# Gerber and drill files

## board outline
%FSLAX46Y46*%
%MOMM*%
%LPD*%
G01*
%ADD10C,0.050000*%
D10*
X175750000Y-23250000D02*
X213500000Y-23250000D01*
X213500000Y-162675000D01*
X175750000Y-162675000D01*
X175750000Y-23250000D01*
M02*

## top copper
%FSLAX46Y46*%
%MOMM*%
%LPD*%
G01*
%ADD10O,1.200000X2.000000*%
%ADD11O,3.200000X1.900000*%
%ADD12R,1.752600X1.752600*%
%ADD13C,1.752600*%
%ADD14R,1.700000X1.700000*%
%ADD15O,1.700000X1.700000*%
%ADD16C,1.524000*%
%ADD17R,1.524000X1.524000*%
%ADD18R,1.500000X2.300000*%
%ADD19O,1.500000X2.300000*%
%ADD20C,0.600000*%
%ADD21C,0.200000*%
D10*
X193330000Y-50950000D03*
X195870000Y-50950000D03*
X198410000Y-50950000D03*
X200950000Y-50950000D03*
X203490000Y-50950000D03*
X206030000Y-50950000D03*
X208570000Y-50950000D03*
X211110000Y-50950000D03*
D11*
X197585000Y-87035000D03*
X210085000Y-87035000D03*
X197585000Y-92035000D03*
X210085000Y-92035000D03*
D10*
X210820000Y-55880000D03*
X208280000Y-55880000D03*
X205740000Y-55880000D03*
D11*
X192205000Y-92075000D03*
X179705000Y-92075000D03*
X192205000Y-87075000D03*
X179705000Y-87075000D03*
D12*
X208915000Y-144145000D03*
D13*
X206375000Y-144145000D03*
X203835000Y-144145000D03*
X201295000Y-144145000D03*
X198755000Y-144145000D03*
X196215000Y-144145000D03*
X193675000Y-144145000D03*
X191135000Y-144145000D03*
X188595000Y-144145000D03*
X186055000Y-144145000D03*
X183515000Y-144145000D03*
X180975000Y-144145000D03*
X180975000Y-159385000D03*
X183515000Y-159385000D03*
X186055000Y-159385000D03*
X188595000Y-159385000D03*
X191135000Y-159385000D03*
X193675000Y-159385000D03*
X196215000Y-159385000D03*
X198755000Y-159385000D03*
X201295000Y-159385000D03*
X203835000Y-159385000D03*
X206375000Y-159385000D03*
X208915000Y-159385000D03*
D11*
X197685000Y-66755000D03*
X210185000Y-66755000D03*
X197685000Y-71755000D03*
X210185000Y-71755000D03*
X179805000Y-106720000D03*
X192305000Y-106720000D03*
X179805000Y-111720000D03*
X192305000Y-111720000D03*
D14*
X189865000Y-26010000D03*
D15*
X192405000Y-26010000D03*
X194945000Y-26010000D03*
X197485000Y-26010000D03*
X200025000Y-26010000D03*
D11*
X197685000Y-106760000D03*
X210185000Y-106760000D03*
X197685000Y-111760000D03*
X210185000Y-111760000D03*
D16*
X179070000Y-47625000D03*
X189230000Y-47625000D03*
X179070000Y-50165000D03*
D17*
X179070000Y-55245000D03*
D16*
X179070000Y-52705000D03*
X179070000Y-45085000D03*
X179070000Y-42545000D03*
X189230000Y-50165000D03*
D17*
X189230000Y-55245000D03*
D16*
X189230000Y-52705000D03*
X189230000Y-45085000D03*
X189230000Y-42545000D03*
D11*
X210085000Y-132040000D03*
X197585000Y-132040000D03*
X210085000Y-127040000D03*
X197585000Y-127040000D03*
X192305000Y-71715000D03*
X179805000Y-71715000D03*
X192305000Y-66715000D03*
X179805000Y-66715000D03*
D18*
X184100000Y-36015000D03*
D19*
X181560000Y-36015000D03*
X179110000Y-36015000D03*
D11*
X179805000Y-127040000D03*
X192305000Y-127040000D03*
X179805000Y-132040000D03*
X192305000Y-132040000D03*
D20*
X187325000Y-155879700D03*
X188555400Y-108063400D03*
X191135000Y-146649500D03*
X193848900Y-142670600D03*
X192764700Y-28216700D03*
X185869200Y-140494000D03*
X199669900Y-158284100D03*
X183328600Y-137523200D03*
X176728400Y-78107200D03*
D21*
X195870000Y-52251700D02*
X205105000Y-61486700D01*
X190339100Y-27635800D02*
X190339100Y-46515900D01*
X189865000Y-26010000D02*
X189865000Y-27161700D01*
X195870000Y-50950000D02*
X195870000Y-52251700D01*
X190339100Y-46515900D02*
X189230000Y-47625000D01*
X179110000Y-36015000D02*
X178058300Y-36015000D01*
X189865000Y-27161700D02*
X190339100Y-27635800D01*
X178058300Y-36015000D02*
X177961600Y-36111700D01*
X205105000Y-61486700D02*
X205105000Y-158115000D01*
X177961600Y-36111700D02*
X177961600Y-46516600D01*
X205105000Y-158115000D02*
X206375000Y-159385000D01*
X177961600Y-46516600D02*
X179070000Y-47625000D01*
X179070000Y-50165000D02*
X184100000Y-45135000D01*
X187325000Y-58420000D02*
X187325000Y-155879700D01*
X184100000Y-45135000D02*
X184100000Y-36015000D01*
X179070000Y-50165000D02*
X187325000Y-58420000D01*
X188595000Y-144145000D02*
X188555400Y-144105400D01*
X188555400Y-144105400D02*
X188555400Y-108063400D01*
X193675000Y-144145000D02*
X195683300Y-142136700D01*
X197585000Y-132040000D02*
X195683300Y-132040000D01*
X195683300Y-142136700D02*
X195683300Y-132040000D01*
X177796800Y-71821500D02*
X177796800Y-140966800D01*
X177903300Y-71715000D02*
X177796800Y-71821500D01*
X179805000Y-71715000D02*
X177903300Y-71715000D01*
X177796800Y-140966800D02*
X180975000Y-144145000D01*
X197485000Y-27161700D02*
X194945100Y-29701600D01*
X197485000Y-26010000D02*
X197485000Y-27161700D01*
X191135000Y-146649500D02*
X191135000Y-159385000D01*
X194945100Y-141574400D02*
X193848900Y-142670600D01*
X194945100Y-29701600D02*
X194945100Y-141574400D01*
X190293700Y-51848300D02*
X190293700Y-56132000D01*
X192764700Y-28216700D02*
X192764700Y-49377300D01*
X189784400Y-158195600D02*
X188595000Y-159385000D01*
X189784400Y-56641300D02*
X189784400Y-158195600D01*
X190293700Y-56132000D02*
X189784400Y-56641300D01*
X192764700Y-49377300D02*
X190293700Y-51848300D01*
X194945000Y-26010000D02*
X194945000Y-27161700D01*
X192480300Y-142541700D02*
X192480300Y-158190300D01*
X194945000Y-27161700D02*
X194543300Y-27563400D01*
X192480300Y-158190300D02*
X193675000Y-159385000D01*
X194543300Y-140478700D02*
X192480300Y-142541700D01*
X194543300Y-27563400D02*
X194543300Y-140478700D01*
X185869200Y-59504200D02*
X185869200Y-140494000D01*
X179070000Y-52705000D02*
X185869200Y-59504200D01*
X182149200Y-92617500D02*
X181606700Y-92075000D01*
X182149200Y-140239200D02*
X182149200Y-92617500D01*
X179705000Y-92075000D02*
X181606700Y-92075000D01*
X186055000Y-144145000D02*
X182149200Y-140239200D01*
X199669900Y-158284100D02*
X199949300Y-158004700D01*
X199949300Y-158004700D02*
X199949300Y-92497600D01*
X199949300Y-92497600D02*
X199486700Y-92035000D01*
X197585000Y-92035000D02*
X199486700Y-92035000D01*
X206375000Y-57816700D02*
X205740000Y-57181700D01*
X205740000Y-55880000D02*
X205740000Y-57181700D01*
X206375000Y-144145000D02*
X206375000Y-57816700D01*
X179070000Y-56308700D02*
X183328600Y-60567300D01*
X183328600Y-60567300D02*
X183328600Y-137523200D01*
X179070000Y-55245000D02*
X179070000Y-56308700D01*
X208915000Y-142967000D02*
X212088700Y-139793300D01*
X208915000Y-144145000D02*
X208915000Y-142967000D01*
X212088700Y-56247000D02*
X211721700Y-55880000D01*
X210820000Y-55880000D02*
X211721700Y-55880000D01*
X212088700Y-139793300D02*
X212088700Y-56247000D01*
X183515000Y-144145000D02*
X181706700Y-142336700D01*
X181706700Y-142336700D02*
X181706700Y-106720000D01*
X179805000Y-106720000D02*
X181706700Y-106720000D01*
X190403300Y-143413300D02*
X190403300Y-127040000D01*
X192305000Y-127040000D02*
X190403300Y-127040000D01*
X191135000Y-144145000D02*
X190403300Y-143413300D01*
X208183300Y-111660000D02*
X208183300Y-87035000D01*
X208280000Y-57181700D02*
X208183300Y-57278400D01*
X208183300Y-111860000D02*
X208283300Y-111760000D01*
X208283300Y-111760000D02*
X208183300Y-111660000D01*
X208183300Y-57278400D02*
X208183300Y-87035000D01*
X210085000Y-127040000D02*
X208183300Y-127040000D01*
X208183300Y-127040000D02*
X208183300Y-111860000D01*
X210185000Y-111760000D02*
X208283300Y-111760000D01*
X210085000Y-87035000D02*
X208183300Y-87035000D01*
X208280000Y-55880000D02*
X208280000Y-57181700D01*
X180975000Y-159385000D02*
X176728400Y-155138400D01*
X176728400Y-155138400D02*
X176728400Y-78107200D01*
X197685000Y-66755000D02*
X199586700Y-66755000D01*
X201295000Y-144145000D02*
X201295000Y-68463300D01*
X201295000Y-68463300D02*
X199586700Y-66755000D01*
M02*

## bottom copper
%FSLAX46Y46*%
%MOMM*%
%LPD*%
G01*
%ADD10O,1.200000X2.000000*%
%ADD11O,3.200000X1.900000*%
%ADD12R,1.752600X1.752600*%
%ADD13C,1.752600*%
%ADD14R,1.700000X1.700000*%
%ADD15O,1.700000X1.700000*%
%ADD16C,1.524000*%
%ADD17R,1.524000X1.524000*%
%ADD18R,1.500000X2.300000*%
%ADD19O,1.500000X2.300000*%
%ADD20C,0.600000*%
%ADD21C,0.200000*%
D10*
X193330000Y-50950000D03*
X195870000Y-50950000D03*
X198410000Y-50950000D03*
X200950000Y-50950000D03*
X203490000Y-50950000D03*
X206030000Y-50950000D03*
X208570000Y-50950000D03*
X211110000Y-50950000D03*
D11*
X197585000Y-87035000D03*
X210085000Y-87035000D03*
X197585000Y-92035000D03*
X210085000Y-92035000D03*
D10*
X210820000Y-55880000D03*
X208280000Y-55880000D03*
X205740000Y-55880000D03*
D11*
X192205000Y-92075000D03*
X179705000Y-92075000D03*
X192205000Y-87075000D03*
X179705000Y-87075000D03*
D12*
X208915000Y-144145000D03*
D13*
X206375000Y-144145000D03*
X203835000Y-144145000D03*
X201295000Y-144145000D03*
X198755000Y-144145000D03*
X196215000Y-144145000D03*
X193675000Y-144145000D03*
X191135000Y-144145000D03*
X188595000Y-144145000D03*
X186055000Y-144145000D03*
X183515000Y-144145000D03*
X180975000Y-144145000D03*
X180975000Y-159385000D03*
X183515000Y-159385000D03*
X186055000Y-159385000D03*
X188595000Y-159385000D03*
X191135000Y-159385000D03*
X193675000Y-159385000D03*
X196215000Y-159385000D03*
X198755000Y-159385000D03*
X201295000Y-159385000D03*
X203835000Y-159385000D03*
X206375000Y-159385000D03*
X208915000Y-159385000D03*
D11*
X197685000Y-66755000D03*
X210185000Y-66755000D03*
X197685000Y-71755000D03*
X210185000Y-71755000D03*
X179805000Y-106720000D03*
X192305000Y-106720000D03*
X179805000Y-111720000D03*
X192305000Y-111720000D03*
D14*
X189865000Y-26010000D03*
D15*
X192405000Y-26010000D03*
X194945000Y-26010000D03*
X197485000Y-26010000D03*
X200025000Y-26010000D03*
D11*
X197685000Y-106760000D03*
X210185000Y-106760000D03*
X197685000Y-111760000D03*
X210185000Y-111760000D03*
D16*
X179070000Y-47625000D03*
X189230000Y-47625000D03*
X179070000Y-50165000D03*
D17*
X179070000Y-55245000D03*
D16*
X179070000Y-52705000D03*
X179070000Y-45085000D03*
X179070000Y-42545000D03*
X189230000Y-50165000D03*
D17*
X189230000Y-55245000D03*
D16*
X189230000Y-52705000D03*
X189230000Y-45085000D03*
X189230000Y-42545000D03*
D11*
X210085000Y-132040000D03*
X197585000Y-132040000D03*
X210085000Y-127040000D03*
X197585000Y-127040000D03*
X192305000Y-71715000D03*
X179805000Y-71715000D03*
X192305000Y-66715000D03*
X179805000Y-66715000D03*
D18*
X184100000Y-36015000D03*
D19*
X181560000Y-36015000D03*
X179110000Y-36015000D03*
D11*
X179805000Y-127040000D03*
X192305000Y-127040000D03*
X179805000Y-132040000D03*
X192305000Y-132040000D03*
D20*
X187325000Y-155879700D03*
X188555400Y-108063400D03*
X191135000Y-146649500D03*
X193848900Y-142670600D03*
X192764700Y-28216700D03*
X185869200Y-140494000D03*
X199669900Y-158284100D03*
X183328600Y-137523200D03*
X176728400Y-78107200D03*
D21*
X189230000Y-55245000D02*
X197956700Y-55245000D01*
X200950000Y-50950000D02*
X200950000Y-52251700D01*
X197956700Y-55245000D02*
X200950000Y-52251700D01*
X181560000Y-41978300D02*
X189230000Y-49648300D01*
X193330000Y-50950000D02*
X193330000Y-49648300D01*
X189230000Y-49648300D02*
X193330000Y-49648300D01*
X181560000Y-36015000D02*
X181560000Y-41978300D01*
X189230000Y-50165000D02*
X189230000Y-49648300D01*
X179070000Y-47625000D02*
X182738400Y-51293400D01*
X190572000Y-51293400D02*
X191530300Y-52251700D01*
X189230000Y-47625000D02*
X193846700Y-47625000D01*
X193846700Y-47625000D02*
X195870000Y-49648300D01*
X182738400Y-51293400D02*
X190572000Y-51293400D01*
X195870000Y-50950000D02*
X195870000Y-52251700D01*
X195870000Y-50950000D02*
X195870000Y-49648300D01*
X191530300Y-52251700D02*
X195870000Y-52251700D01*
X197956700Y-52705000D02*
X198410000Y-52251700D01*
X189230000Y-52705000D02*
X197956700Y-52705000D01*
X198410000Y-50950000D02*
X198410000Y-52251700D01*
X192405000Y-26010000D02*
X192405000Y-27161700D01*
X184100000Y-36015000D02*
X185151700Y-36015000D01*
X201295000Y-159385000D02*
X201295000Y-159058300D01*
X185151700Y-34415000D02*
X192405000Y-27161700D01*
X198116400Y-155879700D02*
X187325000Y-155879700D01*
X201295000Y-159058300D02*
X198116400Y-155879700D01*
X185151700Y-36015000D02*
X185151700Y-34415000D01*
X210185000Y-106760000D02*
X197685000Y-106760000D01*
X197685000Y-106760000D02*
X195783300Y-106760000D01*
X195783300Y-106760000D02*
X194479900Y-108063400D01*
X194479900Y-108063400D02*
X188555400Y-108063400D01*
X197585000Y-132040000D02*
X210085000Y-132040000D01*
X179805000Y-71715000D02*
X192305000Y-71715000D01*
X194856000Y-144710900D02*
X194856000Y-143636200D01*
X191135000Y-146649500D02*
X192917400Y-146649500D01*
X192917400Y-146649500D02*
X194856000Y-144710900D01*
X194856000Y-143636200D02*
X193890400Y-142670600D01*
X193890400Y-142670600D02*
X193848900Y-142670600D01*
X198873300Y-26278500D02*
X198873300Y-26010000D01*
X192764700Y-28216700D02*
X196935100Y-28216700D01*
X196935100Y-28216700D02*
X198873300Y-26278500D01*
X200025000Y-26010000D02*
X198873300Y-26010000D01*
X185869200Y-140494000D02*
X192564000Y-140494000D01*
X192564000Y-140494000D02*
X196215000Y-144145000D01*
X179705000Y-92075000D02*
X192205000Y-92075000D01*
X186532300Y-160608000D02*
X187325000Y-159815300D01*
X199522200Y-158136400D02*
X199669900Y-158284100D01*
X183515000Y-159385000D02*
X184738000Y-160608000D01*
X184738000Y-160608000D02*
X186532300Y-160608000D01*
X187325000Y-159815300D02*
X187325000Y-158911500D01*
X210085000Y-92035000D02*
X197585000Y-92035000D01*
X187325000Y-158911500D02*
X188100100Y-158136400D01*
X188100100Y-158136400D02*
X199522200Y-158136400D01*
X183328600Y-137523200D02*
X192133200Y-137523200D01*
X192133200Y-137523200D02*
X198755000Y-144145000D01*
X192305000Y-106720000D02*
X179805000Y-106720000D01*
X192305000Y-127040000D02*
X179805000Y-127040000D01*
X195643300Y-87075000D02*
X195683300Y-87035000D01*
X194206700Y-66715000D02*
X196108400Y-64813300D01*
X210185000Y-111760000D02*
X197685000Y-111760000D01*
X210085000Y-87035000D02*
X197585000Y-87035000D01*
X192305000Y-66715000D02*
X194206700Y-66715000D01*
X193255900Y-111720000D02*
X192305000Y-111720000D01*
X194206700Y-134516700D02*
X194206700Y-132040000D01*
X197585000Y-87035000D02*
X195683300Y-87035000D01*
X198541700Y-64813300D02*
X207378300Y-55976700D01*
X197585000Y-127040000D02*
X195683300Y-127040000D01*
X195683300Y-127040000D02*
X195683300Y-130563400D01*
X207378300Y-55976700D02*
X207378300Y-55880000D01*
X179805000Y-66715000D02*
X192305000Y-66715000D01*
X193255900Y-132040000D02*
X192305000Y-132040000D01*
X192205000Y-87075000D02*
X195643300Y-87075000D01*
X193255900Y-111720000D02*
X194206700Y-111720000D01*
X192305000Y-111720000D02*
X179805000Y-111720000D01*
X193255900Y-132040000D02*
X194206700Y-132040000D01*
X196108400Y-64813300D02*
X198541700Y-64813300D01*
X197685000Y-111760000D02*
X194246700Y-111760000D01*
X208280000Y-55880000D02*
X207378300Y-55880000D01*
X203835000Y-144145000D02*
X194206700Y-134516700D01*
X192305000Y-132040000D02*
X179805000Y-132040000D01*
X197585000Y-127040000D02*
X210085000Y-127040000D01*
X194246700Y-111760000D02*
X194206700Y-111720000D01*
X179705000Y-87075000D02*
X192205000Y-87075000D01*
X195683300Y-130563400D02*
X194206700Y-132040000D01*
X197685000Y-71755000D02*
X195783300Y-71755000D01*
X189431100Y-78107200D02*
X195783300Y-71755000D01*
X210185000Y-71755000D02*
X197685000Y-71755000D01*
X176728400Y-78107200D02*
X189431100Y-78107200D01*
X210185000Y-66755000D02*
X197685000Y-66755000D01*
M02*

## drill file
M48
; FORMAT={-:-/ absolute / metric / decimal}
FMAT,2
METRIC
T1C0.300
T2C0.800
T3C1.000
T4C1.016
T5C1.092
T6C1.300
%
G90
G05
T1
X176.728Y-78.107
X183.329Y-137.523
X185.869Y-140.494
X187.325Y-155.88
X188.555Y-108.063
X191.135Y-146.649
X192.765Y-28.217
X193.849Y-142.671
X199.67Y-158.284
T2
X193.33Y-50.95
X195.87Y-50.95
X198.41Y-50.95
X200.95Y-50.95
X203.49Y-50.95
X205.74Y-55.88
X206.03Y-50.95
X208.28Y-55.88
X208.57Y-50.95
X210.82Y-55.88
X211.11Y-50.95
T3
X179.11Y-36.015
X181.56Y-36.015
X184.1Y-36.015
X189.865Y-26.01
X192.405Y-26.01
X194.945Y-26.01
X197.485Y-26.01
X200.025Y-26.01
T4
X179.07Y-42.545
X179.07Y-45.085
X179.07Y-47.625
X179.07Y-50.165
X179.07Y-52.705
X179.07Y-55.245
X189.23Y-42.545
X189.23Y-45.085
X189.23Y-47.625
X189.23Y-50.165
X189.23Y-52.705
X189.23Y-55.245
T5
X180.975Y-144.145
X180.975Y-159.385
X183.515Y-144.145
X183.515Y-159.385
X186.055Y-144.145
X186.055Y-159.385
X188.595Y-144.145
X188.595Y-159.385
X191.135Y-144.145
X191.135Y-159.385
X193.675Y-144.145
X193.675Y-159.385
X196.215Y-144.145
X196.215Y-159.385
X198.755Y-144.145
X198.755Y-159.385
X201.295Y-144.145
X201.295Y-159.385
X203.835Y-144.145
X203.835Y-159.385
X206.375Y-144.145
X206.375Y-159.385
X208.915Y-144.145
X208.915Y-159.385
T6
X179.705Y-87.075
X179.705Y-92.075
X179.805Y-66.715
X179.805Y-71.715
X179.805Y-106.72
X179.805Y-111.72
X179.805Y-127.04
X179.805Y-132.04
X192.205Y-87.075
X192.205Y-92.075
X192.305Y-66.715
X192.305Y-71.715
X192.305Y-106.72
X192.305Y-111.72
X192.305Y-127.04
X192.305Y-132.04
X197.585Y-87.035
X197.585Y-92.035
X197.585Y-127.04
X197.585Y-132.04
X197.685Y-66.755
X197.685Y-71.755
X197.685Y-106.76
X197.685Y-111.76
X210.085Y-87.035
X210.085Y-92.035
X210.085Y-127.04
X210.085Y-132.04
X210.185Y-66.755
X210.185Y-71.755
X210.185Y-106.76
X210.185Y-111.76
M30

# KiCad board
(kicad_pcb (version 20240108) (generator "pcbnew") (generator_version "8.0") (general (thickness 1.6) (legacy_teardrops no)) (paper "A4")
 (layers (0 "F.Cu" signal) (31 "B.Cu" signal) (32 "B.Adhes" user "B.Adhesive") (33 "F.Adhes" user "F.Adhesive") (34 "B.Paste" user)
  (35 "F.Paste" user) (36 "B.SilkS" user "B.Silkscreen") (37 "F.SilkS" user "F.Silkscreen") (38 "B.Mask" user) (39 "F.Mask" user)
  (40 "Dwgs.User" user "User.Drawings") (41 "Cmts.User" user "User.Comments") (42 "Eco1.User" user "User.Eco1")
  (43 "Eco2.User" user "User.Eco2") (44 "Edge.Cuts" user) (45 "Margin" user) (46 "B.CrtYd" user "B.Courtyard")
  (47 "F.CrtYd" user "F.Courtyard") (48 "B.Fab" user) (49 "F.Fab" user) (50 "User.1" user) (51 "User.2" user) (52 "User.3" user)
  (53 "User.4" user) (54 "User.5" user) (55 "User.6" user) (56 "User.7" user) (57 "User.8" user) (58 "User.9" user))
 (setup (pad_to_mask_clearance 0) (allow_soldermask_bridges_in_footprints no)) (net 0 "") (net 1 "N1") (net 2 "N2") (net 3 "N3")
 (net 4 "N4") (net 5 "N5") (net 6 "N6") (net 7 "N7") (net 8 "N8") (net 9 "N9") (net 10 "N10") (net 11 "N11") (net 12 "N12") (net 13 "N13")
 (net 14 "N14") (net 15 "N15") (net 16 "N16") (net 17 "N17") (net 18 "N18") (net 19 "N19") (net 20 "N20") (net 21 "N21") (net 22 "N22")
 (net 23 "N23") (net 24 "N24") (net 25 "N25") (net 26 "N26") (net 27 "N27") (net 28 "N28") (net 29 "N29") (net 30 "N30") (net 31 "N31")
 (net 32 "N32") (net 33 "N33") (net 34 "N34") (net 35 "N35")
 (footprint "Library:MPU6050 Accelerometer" (layer "F.Cu") (at 204.47 44.45 90)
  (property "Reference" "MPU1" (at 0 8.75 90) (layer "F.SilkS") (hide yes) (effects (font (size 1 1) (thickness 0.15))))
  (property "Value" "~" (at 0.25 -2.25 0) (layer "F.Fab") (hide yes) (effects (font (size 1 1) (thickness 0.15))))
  (pad "1" thru_hole oval (at -6.5 -11.14) (size 1.2 2) (drill 0.8) (layers "*.Cu" "*.Mask") (remove_unused_layers no) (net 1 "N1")
   (thermal_bridge_angle 45))
  (pad "2" thru_hole oval (at -6.5 -8.6) (size 1.2 2) (drill 0.8) (layers "*.Cu" "*.Mask") (remove_unused_layers no) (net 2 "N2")
   (thermal_bridge_angle 45))
  (pad "3" thru_hole oval (at -6.5 -6.06) (size 1.2 2) (drill 0.8) (layers "*.Cu" "*.Mask") (remove_unused_layers no) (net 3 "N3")
   (thermal_bridge_angle 45))
  (pad "4" thru_hole oval (at -6.5 -3.52) (size 1.2 2) (drill 0.8) (layers "*.Cu" "*.Mask") (remove_unused_layers no) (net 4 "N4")
   (thermal_bridge_angle 45))
  (pad "5" thru_hole oval (at -6.5 -0.98) (size 1.2 2) (drill 0.8) (layers "*.Cu" "*.Mask") (remove_unused_layers no) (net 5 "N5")
   (thermal_bridge_angle 45))
  (pad "6" thru_hole oval (at -6.5 1.56) (size 1.2 2) (drill 0.8) (layers "*.Cu" "*.Mask") (remove_unused_layers no) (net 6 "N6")
   (thermal_bridge_angle 45))
  (pad "7" thru_hole oval (at -6.5 4.1) (size 1.2 2) (drill 0.8) (layers "*.Cu" "*.Mask") (remove_unused_layers no) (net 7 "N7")
   (thermal_bridge_angle 45))
  (pad "8" thru_hole oval (at -6.5 6.64) (size 1.2 2) (drill 0.8) (layers "*.Cu" "*.Mask") (remove_unused_layers no) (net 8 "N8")
   (thermal_bridge_angle 45)))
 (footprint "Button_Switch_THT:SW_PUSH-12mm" (layer "F.Cu") (at 197.585 87.035)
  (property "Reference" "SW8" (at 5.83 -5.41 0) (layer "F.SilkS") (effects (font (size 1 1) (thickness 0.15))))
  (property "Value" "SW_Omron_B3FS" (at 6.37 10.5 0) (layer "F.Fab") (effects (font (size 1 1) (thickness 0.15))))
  (pad "1" thru_hole oval (at 0 0) (size 3.2 1.9) (drill 1.3) (layers "*.Cu" "*.Mask") (remove_unused_layers no) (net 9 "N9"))
  (pad "1" thru_hole oval (at 12.5 0) (size 3.2 1.9) (drill 1.3) (layers "*.Cu" "*.Mask") (remove_unused_layers no) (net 9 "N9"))
  (pad "2" thru_hole oval (at 0 5) (size 3.2 1.9) (drill 1.3) (layers "*.Cu" "*.Mask") (remove_unused_layers no) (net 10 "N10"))
  (pad "2" thru_hole oval (at 12.5 5) (size 3.2 1.9) (drill 1.3) (layers "*.Cu" "*.Mask") (remove_unused_layers no) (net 10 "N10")))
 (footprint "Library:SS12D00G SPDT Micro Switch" (layer "F.Cu") (at 208.28 55.88 180)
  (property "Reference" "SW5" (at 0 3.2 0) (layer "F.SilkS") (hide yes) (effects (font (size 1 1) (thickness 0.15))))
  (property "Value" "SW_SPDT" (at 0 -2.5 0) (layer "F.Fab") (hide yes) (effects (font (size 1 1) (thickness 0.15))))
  (pad "1" thru_hole oval (at -2.54 0 180) (size 1.2 2) (drill 0.8) (layers "*.Cu" "*.Mask") (remove_unused_layers no) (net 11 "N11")
   (thermal_bridge_angle 45))
  (pad "2" thru_hole oval (at 0 0 180) (size 1.2 2) (drill 0.8) (layers "*.Cu" "*.Mask") (remove_unused_layers no) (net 9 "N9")
   (thermal_bridge_angle 45))
  (pad "3" thru_hole oval (at 2.54 0 180) (size 1.2 2) (drill 0.8) (layers "*.Cu" "*.Mask") (remove_unused_layers no) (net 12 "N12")
   (thermal_bridge_angle 45)))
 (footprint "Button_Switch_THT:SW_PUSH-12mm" (layer "F.Cu") (at 192.205 92.075 180)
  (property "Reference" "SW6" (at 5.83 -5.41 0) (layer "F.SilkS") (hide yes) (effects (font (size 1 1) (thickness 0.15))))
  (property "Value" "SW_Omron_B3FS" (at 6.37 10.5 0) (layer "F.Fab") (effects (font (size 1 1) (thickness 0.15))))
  (pad "1" thru_hole oval (at 0 0 180) (size 3.2 1.9) (drill 1.3) (layers "*.Cu" "*.Mask") (remove_unused_layers no) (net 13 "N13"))
  (pad "1" thru_hole oval (at 12.5 0 180) (size 3.2 1.9) (drill 1.3) (layers "*.Cu" "*.Mask") (remove_unused_layers no) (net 13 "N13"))
  (pad "2" thru_hole oval (at 0 5 180) (size 3.2 1.9) (drill 1.3) (layers "*.Cu" "*.Mask") (remove_unused_layers no) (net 9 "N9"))
  (pad "2" thru_hole oval (at 12.5 5 180) (size 3.2 1.9) (drill 1.3) (layers "*.Cu" "*.Mask") (remove_unused_layers no) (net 9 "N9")))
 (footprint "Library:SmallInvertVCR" (layer "F.Cu") (at 207.645 29.845)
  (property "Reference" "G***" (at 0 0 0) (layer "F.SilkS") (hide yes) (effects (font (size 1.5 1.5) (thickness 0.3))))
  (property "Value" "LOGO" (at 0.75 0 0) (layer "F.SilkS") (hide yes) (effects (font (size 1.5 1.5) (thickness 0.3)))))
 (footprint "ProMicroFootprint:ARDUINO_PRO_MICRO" (layer "F.Cu") (at 194.945 151.765 180)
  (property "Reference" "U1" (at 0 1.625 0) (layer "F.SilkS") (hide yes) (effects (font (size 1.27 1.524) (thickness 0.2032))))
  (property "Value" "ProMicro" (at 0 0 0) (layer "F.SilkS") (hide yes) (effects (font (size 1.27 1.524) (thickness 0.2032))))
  (pad "1" thru_hole rect (at -13.97 7.62 180) (size 1.7526 1.7526) (drill 1.0922) (layers "*.Cu" "*.SilkS" "*.Mask")
   (remove_unused_layers no) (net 11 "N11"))
  (pad "2" thru_hole circle (at -11.43 7.62 180) (size 1.7526 1.7526) (drill 1.0922) (layers "*.Cu" "*.SilkS" "*.Mask")
   (remove_unused_layers no) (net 12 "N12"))
  (pad "3" thru_hole circle (at -8.89 7.62 180) (size 1.7526 1.7526) (drill 1.0922) (layers "*.Cu" "*.SilkS" "*.Mask")
   (remove_unused_layers no) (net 9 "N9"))
  (pad "4" thru_hole circle (at -6.35 7.62 180) (size 1.7526 1.7526) (drill 1.0922) (layers "*.Cu" "*.SilkS" "*.Mask")
   (remove_unused_layers no) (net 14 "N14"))
  (pad "5" thru_hole circle (at -3.81 7.62 180) (size 1.7526 1.7526) (drill 1.0922) (layers "*.Cu" "*.SilkS" "*.Mask")
   (remove_unused_layers no) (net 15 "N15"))
  (pad "6" thru_hole circle (at -1.27 7.62 180) (size 1.7526 1.7526) (drill 1.0922) (layers "*.Cu" "*.SilkS" "*.Mask")
   (remove_unused_layers no) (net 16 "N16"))
  (pad "7" thru_hole circle (at 1.27 7.62 180) (size 1.7526 1.7526) (drill 1.0922) (layers "*.Cu" "*.SilkS" "*.Mask")
   (remove_unused_layers no) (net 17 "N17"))
  (pad "8" thru_hole circle (at 3.81 7.62 180) (size 1.7526 1.7526) (drill 1.0922) (layers "*.Cu" "*.SilkS" "*.Mask")
   (remove_unused_layers no) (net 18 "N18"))
  (pad "9" thru_hole circle (at 6.35 7.62 180) (size 1.7526 1.7526) (drill 1.0922) (layers "*.Cu" "*.SilkS" "*.Mask")
   (remove_unused_layers no) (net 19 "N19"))
  (pad "10" thru_hole circle (at 8.89 7.62 180) (size 1.7526 1.7526) (drill 1.0922) (layers "*.Cu" "*.SilkS" "*.Mask")
   (remove_unused_layers no) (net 13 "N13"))
  (pad "11" thru_hole circle (at 11.43 7.62 180) (size 1.7526 1.7526) (drill 1.0922) (layers "*.Cu" "*.SilkS" "*.Mask")
   (remove_unused_layers no) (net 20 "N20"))
  (pad "12" thru_hole circle (at 13.97 7.62 180) (size 1.7526 1.7526) (drill 1.0922) (layers "*.Cu" "*.SilkS" "*.Mask")
   (remove_unused_layers no) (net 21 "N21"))
  (pad "13" thru_hole circle (at 13.97 -7.62 180) (size 1.7526 1.7526) (drill 1.0922) (layers "*.Cu" "*.SilkS" "*.Mask")
   (remove_unused_layers no) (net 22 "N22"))
  (pad "14" thru_hole circle (at 11.43 -7.62 180) (size 1.7526 1.7526) (drill 1.0922) (layers "*.Cu" "*.SilkS" "*.Mask")
   (remove_unused_layers no) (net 10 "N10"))
  (pad "15" thru_hole circle (at 8.89 -7.62 180) (size 1.7526 1.7526) (drill 1.0922) (layers "*.Cu" "*.SilkS" "*.Mask")
   (remove_unused_layers no) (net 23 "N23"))
  (pad "16" thru_hole circle (at 6.35 -7.62 180) (size 1.7526 1.7526) (drill 1.0922) (layers "*.Cu" "*.SilkS" "*.Mask")
   (remove_unused_layers no) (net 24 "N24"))
  (pad "17" thru_hole circle (at 3.81 -7.62 180) (size 1.7526 1.7526) (drill 1.0922) (layers "*.Cu" "*.SilkS" "*.Mask")
   (remove_unused_layers no) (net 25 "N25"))
  (pad "18" thru_hole circle (at 1.27 -7.62 180) (size 1.7526 1.7526) (drill 1.0922) (layers "*.Cu" "*.SilkS" "*.Mask")
   (remove_unused_layers no) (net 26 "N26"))
  (pad "19" thru_hole circle (at -1.27 -7.62 180) (size 1.7526 1.7526) (drill 1.0922) (layers "*.Cu" "*.SilkS" "*.Mask")
   (remove_unused_layers no) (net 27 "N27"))
  (pad "20" thru_hole circle (at -3.81 -7.62 180) (size 1.7526 1.7526) (drill 1.0922) (layers "*.Cu" "*.SilkS" "*.Mask")
   (remove_unused_layers no) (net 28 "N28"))
  (pad "21" thru_hole circle (at -6.35 -7.62 180) (size 1.7526 1.7526) (drill 1.0922) (layers "*.Cu" "*.SilkS" "*.Mask")
   (remove_unused_layers no) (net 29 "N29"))
  (pad "22" thru_hole circle (at -8.89 -7.62 180) (size 1.7526 1.7526) (drill 1.0922) (layers "*.Cu" "*.SilkS" "*.Mask")
   (remove_unused_layers no) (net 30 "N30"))
  (pad "23" thru_hole circle (at -11.43 -7.62 180) (size 1.7526 1.7526) (drill 1.0922) (layers "*.Cu" "*.SilkS" "*.Mask")
   (remove_unused_layers no) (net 2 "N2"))
  (pad "24" thru_hole circle (at -13.97 -7.62 180) (size 1.7526 1.7526) (drill 1.0922) (layers "*.Cu" "*.SilkS" "*.Mask")
   (remove_unused_layers no) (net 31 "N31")))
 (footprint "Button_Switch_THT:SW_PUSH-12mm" (layer "F.Cu") (at 197.685 66.755)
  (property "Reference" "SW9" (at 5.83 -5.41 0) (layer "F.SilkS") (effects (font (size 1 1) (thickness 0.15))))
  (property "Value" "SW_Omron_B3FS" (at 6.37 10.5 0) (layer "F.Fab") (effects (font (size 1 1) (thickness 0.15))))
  (pad "1" thru_hole oval (at 0 0) (size 3.2 1.9) (drill 1.3) (layers "*.Cu" "*.Mask") (remove_unused_layers no) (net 14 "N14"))
  (pad "1" thru_hole oval (at 12.5 0) (size 3.2 1.9) (drill 1.3) (layers "*.Cu" "*.Mask") (remove_unused_layers no) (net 14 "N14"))
  (pad "2" thru_hole oval (at 0 5) (size 3.2 1.9) (drill 1.3) (layers "*.Cu" "*.Mask") (remove_unused_layers no) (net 22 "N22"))
  (pad "2" thru_hole oval (at 12.5 5) (size 3.2 1.9) (drill 1.3) (layers "*.Cu" "*.Mask") (remove_unused_layers no) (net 22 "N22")))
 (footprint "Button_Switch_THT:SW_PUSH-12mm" (layer "F.Cu") (at 179.805 106.72)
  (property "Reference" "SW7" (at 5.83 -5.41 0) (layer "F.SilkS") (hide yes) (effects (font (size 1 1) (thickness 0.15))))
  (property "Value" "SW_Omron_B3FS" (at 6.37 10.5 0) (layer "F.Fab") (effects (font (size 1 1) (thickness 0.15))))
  (pad "1" thru_hole oval (at 0 0) (size 3.2 1.9) (drill 1.3) (layers "*.Cu" "*.Mask") (remove_unused_layers no) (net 20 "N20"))
  (pad "1" thru_hole oval (at 12.5 0) (size 3.2 1.9) (drill 1.3) (layers "*.Cu" "*.Mask") (remove_unused_layers no) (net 20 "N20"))
  (pad "2" thru_hole oval (at 0 5) (size 3.2 1.9) (drill 1.3) (layers "*.Cu" "*.Mask") (remove_unused_layers no) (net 9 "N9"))
  (pad "2" thru_hole oval (at 12.5 5) (size 3.2 1.9) (drill 1.3) (layers "*.Cu" "*.Mask") (remove_unused_layers no) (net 9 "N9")))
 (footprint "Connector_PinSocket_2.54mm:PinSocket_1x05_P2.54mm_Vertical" (layer "F.Cu") (at 189.865 26.01 90)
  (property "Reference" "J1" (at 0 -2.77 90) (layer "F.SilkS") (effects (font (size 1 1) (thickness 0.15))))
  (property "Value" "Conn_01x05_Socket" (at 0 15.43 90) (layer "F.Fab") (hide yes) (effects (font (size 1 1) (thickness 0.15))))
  (pad "1" thru_hole rect (at 0 0 90) (size 1.7 1.7) (drill 1) (layers "*.Cu" "*.Mask") (remove_unused_layers no) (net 2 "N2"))
  (pad "2" thru_hole oval (at 0 2.54 90) (size 1.7 1.7) (drill 1) (layers "*.Cu" "*.Mask") (remove_unused_layers no) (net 29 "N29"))
  (pad "3" thru_hole oval (at 0 5.08 90) (size 1.7 1.7) (drill 1) (layers "*.Cu" "*.Mask") (remove_unused_layers no) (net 26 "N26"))
  (pad "4" thru_hole oval (at 0 7.62 90) (size 1.7 1.7) (drill 1) (layers "*.Cu" "*.Mask") (remove_unused_layers no) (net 25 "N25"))
  (pad "5" thru_hole oval (at 0 10.16 90) (size 1.7 1.7) (drill 1) (layers "*.Cu" "*.Mask") (remove_unused_layers no) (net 24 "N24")))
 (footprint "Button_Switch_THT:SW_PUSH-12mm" (layer "F.Cu") (at 197.685 106.76)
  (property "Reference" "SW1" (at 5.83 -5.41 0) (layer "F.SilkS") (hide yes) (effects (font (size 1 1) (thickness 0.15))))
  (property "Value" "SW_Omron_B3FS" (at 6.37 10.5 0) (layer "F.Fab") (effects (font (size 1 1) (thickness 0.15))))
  (pad "1" thru_hole oval (at 0 0) (size 3.2 1.9) (drill 1.3) (layers "*.Cu" "*.Mask") (remove_unused_layers no) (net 19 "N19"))
  (pad "1" thru_hole oval (at 12.5 0) (size 3.2 1.9) (drill 1.3) (layers "*.Cu" "*.Mask") (remove_unused_layers no) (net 19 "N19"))
  (pad "2" thru_hole oval (at 0 5) (size 3.2 1.9) (drill 1.3) (layers "*.Cu" "*.Mask") (remove_unused_layers no) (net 9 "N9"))
  (pad "2" thru_hole oval (at 12.5 5) (size 3.2 1.9) (drill 1.3) (layers "*.Cu" "*.Mask") (remove_unused_layers no) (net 9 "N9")))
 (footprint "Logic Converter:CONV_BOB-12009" (layer "F.Cu") (at 184.15 48.895 180)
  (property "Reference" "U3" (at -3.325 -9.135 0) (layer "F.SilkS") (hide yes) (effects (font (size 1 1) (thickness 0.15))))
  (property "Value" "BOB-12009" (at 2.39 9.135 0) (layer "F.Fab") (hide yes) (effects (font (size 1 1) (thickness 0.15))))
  (pad "GND_1" thru_hole circle (at 5.08 1.27 180) (size 1.524 1.524) (drill 1.016) (layers "*.Cu" "*.Mask") (remove_unused_layers no)
   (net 2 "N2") (solder_mask_margin 0.102))
  (pad "GND_2" thru_hole circle (at -5.08 1.27 180) (size 1.524 1.524) (drill 1.016) (layers "*.Cu" "*.Mask") (remove_unused_layers no)
   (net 2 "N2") (solder_mask_margin 0.102))
  (pad "HV" thru_hole circle (at 5.08 -1.27 180) (size 1.524 1.524) (drill 1.016) (layers "*.Cu" "*.Mask") (remove_unused_layers no)
   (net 29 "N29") (solder_mask_margin 0.102))
  (pad "HV1" thru_hole rect (at 5.08 -6.35 180) (size 1.524 1.524) (drill 1.016) (layers "*.Cu" "*.Mask") (remove_unused_layers no)
   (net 15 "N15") (solder_mask_margin 0.102))
  (pad "HV2" thru_hole circle (at 5.08 -3.81 180) (size 1.524 1.524) (drill 1.016) (layers "*.Cu" "*.Mask") (remove_unused_layers no)
   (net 16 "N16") (solder_mask_margin 0.102))
  (pad "HV3" thru_hole circle (at 5.08 3.81 180) (size 1.524 1.524) (drill 1.016) (layers "*.Cu" "*.Mask") (remove_unused_layers no)
   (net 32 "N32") (solder_mask_margin 0.102))
  (pad "HV4" thru_hole circle (at 5.08 6.35 180) (size 1.524 1.524) (drill 1.016) (layers "*.Cu" "*.Mask") (remove_unused_layers no)
   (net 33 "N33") (solder_mask_margin 0.102))
  (pad "LV" thru_hole circle (at -5.08 -1.27 180) (size 1.524 1.524) (drill 1.016) (layers "*.Cu" "*.Mask") (remove_unused_layers no)
   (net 1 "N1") (solder_mask_margin 0.102))
  (pad "LV1" thru_hole rect (at -5.08 -6.35 180) (size 1.524 1.524) (drill 1.016) (layers "*.Cu" "*.Mask") (remove_unused_layers no)
   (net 4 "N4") (solder_mask_margin 0.102))
  (pad "LV2" thru_hole circle (at -5.08 -3.81 180) (size 1.524 1.524) (drill 1.016) (layers "*.Cu" "*.Mask") (remove_unused_layers no)
   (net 3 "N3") (solder_mask_margin 0.102))
  (pad "LV3" thru_hole circle (at -5.08 3.81 180) (size 1.524 1.524) (drill 1.016) (layers "*.Cu" "*.Mask") (remove_unused_layers no)
   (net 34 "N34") (solder_mask_margin 0.102))
  (pad "LV4" thru_hole circle (at -5.08 6.35 180) (size 1.524 1.524) (drill 1.016) (layers "*.Cu" "*.Mask") (remove_unused_layers no)
   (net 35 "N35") (solder_mask_margin 0.102)))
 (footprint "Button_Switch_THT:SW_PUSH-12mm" (layer "F.Cu") (at 210.085 132.04 180)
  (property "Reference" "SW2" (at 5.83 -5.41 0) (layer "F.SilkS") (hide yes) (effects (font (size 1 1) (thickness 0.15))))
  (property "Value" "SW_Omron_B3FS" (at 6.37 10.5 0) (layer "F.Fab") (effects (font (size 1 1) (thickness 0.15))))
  (pad "1" thru_hole oval (at 0 0 180) (size 3.2 1.9) (drill 1.3) (layers "*.Cu" "*.Mask") (remove_unused_layers no) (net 17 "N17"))
  (pad "1" thru_hole oval (at 12.5 0 180) (size 3.2 1.9) (drill 1.3) (layers "*.Cu" "*.Mask") (remove_unused_layers no) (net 17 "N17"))
  (pad "2" thru_hole oval (at 0 5 180) (size 3.2 1.9) (drill 1.3) (layers "*.Cu" "*.Mask") (remove_unused_layers no) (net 9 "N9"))
  (pad "2" thru_hole oval (at 12.5 5 180) (size 3.2 1.9) (drill 1.3) (layers "*.Cu" "*.Mask") (remove_unused_layers no) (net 9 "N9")))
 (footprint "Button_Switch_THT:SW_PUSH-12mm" (layer "F.Cu") (at 192.305 71.715 180)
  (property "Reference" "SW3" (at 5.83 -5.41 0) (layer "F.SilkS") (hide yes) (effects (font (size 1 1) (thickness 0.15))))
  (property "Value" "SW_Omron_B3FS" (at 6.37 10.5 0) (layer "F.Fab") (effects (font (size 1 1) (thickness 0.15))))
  (pad "1" thru_hole oval (at 0 0 180) (size 3.2 1.9) (drill 1.3) (layers "*.Cu" "*.Mask") (remove_unused_layers no) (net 21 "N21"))
  (pad "1" thru_hole oval (at 12.5 0 180) (size 3.2 1.9) (drill 1.3) (layers "*.Cu" "*.Mask") (remove_unused_layers no) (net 21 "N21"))
  (pad "2" thru_hole oval (at 0 5 180) (size 3.2 1.9) (drill 1.3) (layers "*.Cu" "*.Mask") (remove_unused_layers no) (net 9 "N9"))
  (pad "2" thru_hole oval (at 12.5 5 180) (size 3.2 1.9) (drill 1.3) (layers "*.Cu" "*.Mask") (remove_unused_layers no) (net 9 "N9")))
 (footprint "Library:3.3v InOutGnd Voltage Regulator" (layer "F.Cu") (at 181.61 37.515)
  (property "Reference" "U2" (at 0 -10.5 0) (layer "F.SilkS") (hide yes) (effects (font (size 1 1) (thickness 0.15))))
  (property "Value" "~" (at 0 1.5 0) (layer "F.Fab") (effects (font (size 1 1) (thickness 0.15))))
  (pad "1" thru_hole rect (at 2.49 -1.5) (size 1.5 2.3) (drill 1) (layers "*.Cu" "*.Mask") (remove_unused_layers no) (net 29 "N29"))
  (pad "2" thru_hole oval (at -0.05 -1.5) (size 1.5 2.3) (drill 1) (layers "*.Cu" "*.Mask") (remove_unused_layers no) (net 1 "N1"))
  (pad "3" thru_hole oval (at -2.5 -1.5) (size 1.5 2.3) (drill 1) (layers "*.Cu" "*.Mask") (remove_unused_layers no) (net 2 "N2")))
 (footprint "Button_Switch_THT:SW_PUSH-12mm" (layer "F.Cu") (at 179.805 127.04)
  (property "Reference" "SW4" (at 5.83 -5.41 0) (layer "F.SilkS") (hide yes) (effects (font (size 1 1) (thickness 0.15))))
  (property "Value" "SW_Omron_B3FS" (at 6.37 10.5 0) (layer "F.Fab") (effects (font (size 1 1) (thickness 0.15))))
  (pad "1" thru_hole oval (at 0 0) (size 3.2 1.9) (drill 1.3) (layers "*.Cu" "*.Mask") (remove_unused_layers no) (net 18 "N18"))
  (pad "1" thru_hole oval (at 12.5 0) (size 3.2 1.9) (drill 1.3) (layers "*.Cu" "*.Mask") (remove_unused_layers no) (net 18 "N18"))
  (pad "2" thru_hole oval (at 0 5) (size 3.2 1.9) (drill 1.3) (layers "*.Cu" "*.Mask") (remove_unused_layers no) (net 9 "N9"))
  (pad "2" thru_hole oval (at 12.5 5) (size 3.2 1.9) (drill 1.3) (layers "*.Cu" "*.Mask") (remove_unused_layers no) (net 9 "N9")))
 (gr_rect (start 175.75 23.25) (end 213.5 162.675) (stroke (width 0.05) (type default)) (fill none) (layer "Edge.Cuts"))
 (segment (start 189.23 55.245) (end 197.9567 55.245) (width 0.2) (layer "B.Cu") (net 4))
 (segment (start 200.95 50.95) (end 200.95 52.2517) (width 0.2) (layer "B.Cu") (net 4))
 (segment (start 197.9567 55.245) (end 200.95 52.2517) (width 0.2) (layer "B.Cu") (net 4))
 (segment (start 181.56 41.9783) (end 189.23 49.6483) (width 0.2) (layer "B.Cu") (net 1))
 (segment (start 193.33 50.95) (end 193.33 49.6483) (width 0.2) (layer "B.Cu") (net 1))
 (segment (start 189.23 49.6483) (end 193.33 49.6483) (width 0.2) (layer "B.Cu") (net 1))
 (segment (start 181.56 36.015) (end 181.56 41.9783) (width 0.2) (layer "B.Cu") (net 1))
 (segment (start 189.23 50.165) (end 189.23 49.6483) (width 0.2) (layer "B.Cu") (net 1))
 (segment (start 195.87 52.2517) (end 205.105 61.4867) (width 0.2) (layer "F.Cu") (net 2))
 (segment (start 190.3391 27.6358) (end 190.3391 46.5159) (width 0.2) (layer "F.Cu") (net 2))
 (segment (start 189.865 26.01) (end 189.865 27.1617) (width 0.2) (layer "F.Cu") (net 2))
 (segment (start 195.87 50.95) (end 195.87 52.2517) (width 0.2) (layer "F.Cu") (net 2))
 (segment (start 190.3391 46.5159) (end 189.23 47.625) (width 0.2) (layer "F.Cu") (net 2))
 (segment (start 179.11 36.015) (end 178.0583 36.015) (width 0.2) (layer "F.Cu") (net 2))
 (segment (start 189.865 27.1617) (end 190.3391 27.6358) (width 0.2) (layer "F.Cu") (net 2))
 (segment (start 178.0583 36.015) (end 177.9616 36.1117) (width 0.2) (layer "F.Cu") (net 2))
 (segment (start 205.105 61.4867) (end 205.105 158.115) (width 0.2) (layer "F.Cu") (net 2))
 (segment (start 177.9616 36.1117) (end 177.9616 46.5166) (width 0.2) (layer "F.Cu") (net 2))
 (segment (start 205.105 158.115) (end 206.375 159.385) (width 0.2) (layer "F.Cu") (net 2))
 (segment (start 177.9616 46.5166) (end 179.07 47.625) (width 0.2) (layer "F.Cu") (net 2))
 (segment (start 179.07 47.625) (end 182.7384 51.2934) (width 0.2) (layer "B.Cu") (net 2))
 (segment (start 190.572 51.2934) (end 191.5303 52.2517) (width 0.2) (layer "B.Cu") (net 2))
 (segment (start 189.23 47.625) (end 193.8467 47.625) (width 0.2) (layer "B.Cu") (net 2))
 (segment (start 193.8467 47.625) (end 195.87 49.6483) (width 0.2) (layer "B.Cu") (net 2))
 (segment (start 182.7384 51.2934) (end 190.572 51.2934) (width 0.2) (layer "B.Cu") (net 2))
 (segment (start 195.87 50.95) (end 195.87 52.2517) (width 0.2) (layer "B.Cu") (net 2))
 (segment (start 195.87 50.95) (end 195.87 49.6483) (width 0.2) (layer "B.Cu") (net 2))
 (segment (start 191.5303 52.2517) (end 195.87 52.2517) (width 0.2) (layer "B.Cu") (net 2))
 (segment (start 197.9567 52.705) (end 198.41 52.2517) (width 0.2) (layer "B.Cu") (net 3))
 (segment (start 189.23 52.705) (end 197.9567 52.705) (width 0.2) (layer "B.Cu") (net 3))
 (segment (start 198.41 50.95) (end 198.41 52.2517) (width 0.2) (layer "B.Cu") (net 3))
 (segment (start 179.07 50.165) (end 184.1 45.135) (width 0.2) (layer "F.Cu") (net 29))
 (segment (start 187.325 58.42) (end 187.325 155.8797) (width 0.2) (layer "F.Cu") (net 29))
 (segment (start 184.1 45.135) (end 184.1 36.015) (width 0.2) (layer "F.Cu") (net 29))
 (segment (start 179.07 50.165) (end 187.325 58.42) (width 0.2) (layer "F.Cu") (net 29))
 (via (at 187.325 155.8797) (size 0.6) (drill 0.3) (layers "F.Cu" "B.Cu") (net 29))
 (segment (start 192.405 26.01) (end 192.405 27.1617) (width 0.2) (layer "B.Cu") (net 29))
 (segment (start 184.1 36.015) (end 185.1517 36.015) (width 0.2) (layer "B.Cu") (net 29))
 (segment (start 201.295 159.385) (end 201.295 159.0583) (width 0.2) (layer "B.Cu") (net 29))
 (segment (start 185.1517 34.415) (end 192.405 27.1617) (width 0.2) (layer "B.Cu") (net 29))
 (segment (start 198.1164 155.8797) (end 187.325 155.8797) (width 0.2) (layer "B.Cu") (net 29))
 (segment (start 201.295 159.0583) (end 198.1164 155.8797) (width 0.2) (layer "B.Cu") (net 29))
 (segment (start 185.1517 36.015) (end 185.1517 34.415) (width 0.2) (layer "B.Cu") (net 29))
 (segment (start 188.595 144.145) (end 188.5554 144.1054) (width 0.2) (layer "F.Cu") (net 19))
 (segment (start 188.5554 144.1054) (end 188.5554 108.0634) (width 0.2) (layer "F.Cu") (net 19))
 (via (at 188.5554 108.0634) (size 0.6) (drill 0.3) (layers "F.Cu" "B.Cu") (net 19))
 (segment (start 210.185 106.76) (end 197.685 106.76) (width 0.2) (layer "B.Cu") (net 19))
 (segment (start 197.685 106.76) (end 195.7833 106.76) (width 0.2) (layer "B.Cu") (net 19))
 (segment (start 195.7833 106.76) (end 194.4799 108.0634) (width 0.2) (layer "B.Cu") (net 19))
 (segment (start 194.4799 108.0634) (end 188.5554 108.0634) (width 0.2) (layer "B.Cu") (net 19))
 (segment (start 193.675 144.145) (end 195.6833 142.1367) (width 0.2) (layer "F.Cu") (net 17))
 (segment (start 197.585 132.04) (end 195.6833 132.04) (width 0.2) (layer "F.Cu") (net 17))
 (segment (start 195.6833 142.1367) (end 195.6833 132.04) (width 0.2) (layer "F.Cu") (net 17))
 (segment (start 197.585 132.04) (end 210.085 132.04) (width 0.2) (layer "B.Cu") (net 17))
 (segment (start 177.7968 71.8215) (end 177.7968 140.9668) (width 0.2) (layer "F.Cu") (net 21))
 (segment (start 177.9033 71.715) (end 177.7968 71.8215) (width 0.2) (layer "F.Cu") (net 21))
 (segment (start 179.805 71.715) (end 177.9033 71.715) (width 0.2) (layer "F.Cu") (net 21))
 (segment (start 177.7968 140.9668) (end 180.975 144.145) (width 0.2) (layer "F.Cu") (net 21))
 (segment (start 179.805 71.715) (end 192.305 71.715) (width 0.2) (layer "B.Cu") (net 21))
 (segment (start 197.485 27.1617) (end 194.9451 29.7016) (width 0.2) (layer "F.Cu") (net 25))
 (segment (start 197.485 26.01) (end 197.485 27.1617) (width 0.2) (layer "F.Cu") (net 25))
 (segment (start 191.135 146.6495) (end 191.135 159.385) (width 0.2) (layer "F.Cu") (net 25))
 (segment (start 194.9451 141.5744) (end 193.8489 142.6706) (width 0.2) (layer "F.Cu") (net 25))
 (segment (start 194.9451 29.7016) (end 194.9451 141.5744) (width 0.2) (layer "F.Cu") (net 25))
 (via (at 191.135 146.6495) (size 0.6) (drill 0.3) (layers "F.Cu" "B.Cu") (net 25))
 (via (at 193.8489 142.6706) (size 0.6) (drill 0.3) (layers "F.Cu" "B.Cu") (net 25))
 (segment (start 194.856 144.7109) (end 194.856 143.6362) (width 0.2) (layer "B.Cu") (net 25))
 (segment (start 191.135 146.6495) (end 192.9174 146.6495) (width 0.2) (layer "B.Cu") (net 25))
 (segment (start 192.9174 146.6495) (end 194.856 144.7109) (width 0.2) (layer "B.Cu") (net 25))
 (segment (start 194.856 143.6362) (end 193.8904 142.6706) (width 0.2) (layer "B.Cu") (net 25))
 (segment (start 193.8904 142.6706) (end 193.8489 142.6706) (width 0.2) (layer "B.Cu") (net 25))
 (segment (start 190.2937 51.8483) (end 190.2937 56.132) (width 0.2) (layer "F.Cu") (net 24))
 (segment (start 192.7647 28.2167) (end 192.7647 49.3773) (width 0.2) (layer "F.Cu") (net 24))
 (segment (start 189.7844 158.1956) (end 188.595 159.385) (width 0.2) (layer "F.Cu") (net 24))
 (segment (start 189.7844 56.6413) (end 189.7844 158.1956) (width 0.2) (layer "F.Cu") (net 24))
 (segment (start 190.2937 56.132) (end 189.7844 56.6413) (width 0.2) (layer "F.Cu") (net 24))
 (segment (start 192.7647 49.3773) (end 190.2937 51.8483) (width 0.2) (layer "F.Cu") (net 24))
 (via (at 192.7647 28.2167) (size 0.6) (drill 0.3) (layers "F.Cu" "B.Cu") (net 24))
 (segment (start 198.8733 26.2785) (end 198.8733 26.01) (width 0.2) (layer "B.Cu") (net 24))
 (segment (start 192.7647 28.2167) (end 196.9351 28.2167) (width 0.2) (layer "B.Cu") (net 24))
 (segment (start 196.9351 28.2167) (end 198.8733 26.2785) (width 0.2) (layer "B.Cu") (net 24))
 (segment (start 200.025 26.01) (end 198.8733 26.01) (width 0.2) (layer "B.Cu") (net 24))
 (segment (start 194.945 26.01) (end 194.945 27.1617) (width 0.2) (layer "F.Cu") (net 26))
 (segment (start 192.4803 142.5417) (end 192.4803 158.1903) (width 0.2) (layer "F.Cu") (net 26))
 (segment (start 194.945 27.1617) (end 194.5433 27.5634) (width 0.2) (layer "F.Cu") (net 26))
 (segment (start 192.4803 158.1903) (end 193.675 159.385) (width 0.2) (layer "F.Cu") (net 26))
 (segment (start 194.5433 140.4787) (end 192.4803 142.5417) (width 0.2) (layer "F.Cu") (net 26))
 (segment (start 194.5433 27.5634) (end 194.5433 140.4787) (width 0.2) (layer "F.Cu") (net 26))
 (segment (start 185.8692 59.5042) (end 185.8692 140.494) (width 0.2) (layer "F.Cu") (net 16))
 (segment (start 179.07 52.705) (end 185.8692 59.5042) (width 0.2) (layer "F.Cu") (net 16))
 (via (at 185.8692 140.494) (size 0.6) (drill 0.3) (layers "F.Cu" "B.Cu") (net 16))
 (segment (start 185.8692 140.494) (end 192.564 140.494) (width 0.2) (layer "B.Cu") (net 16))
 (segment (start 192.564 140.494) (end 196.215 144.145) (width 0.2) (layer "B.Cu") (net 16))
 (segment (start 182.1492 92.6175) (end 181.6067 92.075) (width 0.2) (layer "F.Cu") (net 13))
 (segment (start 182.1492 140.2392) (end 182.1492 92.6175) (width 0.2) (layer "F.Cu") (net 13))
 (segment (start 179.705 92.075) (end 181.6067 92.075) (width 0.2) (layer "F.Cu") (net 13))
 (segment (start 186.055 144.145) (end 182.1492 140.2392) (width 0.2) (layer "F.Cu") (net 13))
 (segment (start 179.705 92.075) (end 192.205 92.075) (width 0.2) (layer "B.Cu") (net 13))
 (segment (start 199.6699 158.2841) (end 199.9493 158.0047) (width 0.2) (layer "F.Cu") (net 10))
 (segment (start 199.9493 158.0047) (end 199.9493 92.4976) (width 0.2) (layer "F.Cu") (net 10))
 (segment (start 199.9493 92.4976) (end 199.4867 92.035) (width 0.2) (layer "F.Cu") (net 10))
 (segment (start 197.585 92.035) (end 199.4867 92.035) (width 0.2) (layer "F.Cu") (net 10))
 (via (at 199.6699 158.2841) (size 0.6) (drill 0.3) (layers "F.Cu" "B.Cu") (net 10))
 (segment (start 186.5323 160.608) (end 187.325 159.8153) (width 0.2) (layer "B.Cu") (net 10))
 (segment (start 199.5222 158.1364) (end 199.6699 158.2841) (width 0.2) (layer "B.Cu") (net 10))
 (segment (start 183.515 159.385) (end 184.738 160.608) (width 0.2) (layer "B.Cu") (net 10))
 (segment (start 184.738 160.608) (end 186.5323 160.608) (width 0.2) (layer "B.Cu") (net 10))
 (segment (start 187.325 159.8153) (end 187.325 158.9115) (width 0.2) (layer "B.Cu") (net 10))
 (segment (start 210.085 92.035) (end 197.585 92.035) (width 0.2) (layer "B.Cu") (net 10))
 (segment (start 187.325 158.9115) (end 188.1001 158.1364) (width 0.2) (layer "B.Cu") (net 10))
 (segment (start 188.1001 158.1364) (end 199.5222 158.1364) (width 0.2) (layer "B.Cu") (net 10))
 (segment (start 206.375 57.8167) (end 205.74 57.1817) (width 0.2) (layer "F.Cu") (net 12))
 (segment (start 205.74 55.88) (end 205.74 57.1817) (width 0.2) (layer "F.Cu") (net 12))
 (segment (start 206.375 144.145) (end 206.375 57.8167) (width 0.2) (layer "F.Cu") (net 12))
 (segment (start 179.07 56.3087) (end 183.3286 60.5673) (width 0.2) (layer "F.Cu") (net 15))
 (segment (start 183.3286 60.5673) (end 183.3286 137.5232) (width 0.2) (layer "F.Cu") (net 15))
 (segment (start 179.07 55.245) (end 179.07 56.3087) (width 0.2) (layer "F.Cu") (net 15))
 (via (at 183.3286 137.5232) (size 0.6) (drill 0.3) (layers "F.Cu" "B.Cu") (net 15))
 (segment (start 183.3286 137.5232) (end 192.1332 137.5232) (width 0.2) (layer "B.Cu") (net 15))
 (segment (start 192.1332 137.5232) (end 198.755 144.145) (width 0.2) (layer "B.Cu") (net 15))
 (segment (start 208.915 142.967) (end 212.0887 139.7933) (width 0.2) (layer "F.Cu") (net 11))
 (segment (start 208.915 144.145) (end 208.915 142.967) (width 0.2) (layer "F.Cu") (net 11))
 (segment (start 212.0887 56.247) (end 211.7217 55.88) (width 0.2) (layer "F.Cu") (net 11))
 (segment (start 210.82 55.88) (end 211.7217 55.88) (width 0.2) (layer "F.Cu") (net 11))
 (segment (start 212.0887 139.7933) (end 212.0887 56.247) (width 0.2) (layer "F.Cu") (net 11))
 (segment (start 183.515 144.145) (end 181.7067 142.3367) (width 0.2) (layer "F.Cu") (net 20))
 (segment (start 181.7067 142.3367) (end 181.7067 106.72) (width 0.2) (layer "F.Cu") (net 20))
 (segment (start 179.805 106.72) (end 181.7067 106.72) (width 0.2) (layer "F.Cu") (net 20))
 (segment (start 192.305 106.72) (end 179.805 106.72) (width 0.2) (layer "B.Cu") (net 20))
 (segment (start 190.4033 143.4133) (end 190.4033 127.04) (width 0.2) (layer "F.Cu") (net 18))
 (segment (start 192.305 127.04) (end 190.4033 127.04) (width 0.2) (layer "F.Cu") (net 18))
 (segment (start 191.135 144.145) (end 190.4033 143.4133) (width 0.2) (layer "F.Cu") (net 18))
 (segment (start 192.305 127.04) (end 179.805 127.04) (width 0.2) (layer "B.Cu") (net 18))
 (segment (start 208.1833 111.66) (end 208.1833 87.035) (width 0.2) (layer "F.Cu") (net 9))
 (segment (start 208.28 57.1817) (end 208.1833 57.2784) (width 0.2) (layer "F.Cu") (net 9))
 (segment (start 208.1833 111.86) (end 208.2833 111.76) (width 0.2) (layer "F.Cu") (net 9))
 (segment (start 208.2833 111.76) (end 208.1833 111.66) (width 0.2) (layer "F.Cu") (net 9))
 (segment (start 208.1833 57.2784) (end 208.1833 87.035) (width 0.2) (layer "F.Cu") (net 9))
 (segment (start 210.085 127.04) (end 208.1833 127.04) (width 0.2) (layer "F.Cu") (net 9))
 (segment (start 208.1833 127.04) (end 208.1833 111.86) (width 0.2) (layer "F.Cu") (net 9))
 (segment (start 210.185 111.76) (end 208.2833 111.76) (width 0.2) (layer "F.Cu") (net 9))
 (segment (start 210.085 87.035) (end 208.1833 87.035) (width 0.2) (layer "F.Cu") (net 9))
 (segment (start 208.28 55.88) (end 208.28 57.1817) (width 0.2) (layer "F.Cu") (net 9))
 (segment (start 195.6433 87.075) (end 195.6833 87.035) (width 0.2) (layer "B.Cu") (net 9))
 (segment (start 194.2067 66.715) (end 196.1084 64.8133) (width 0.2) (layer "B.Cu") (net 9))
 (segment (start 210.185 111.76) (end 197.685 111.76) (width 0.2) (layer "B.Cu") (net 9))
 (segment (start 210.085 87.035) (end 197.585 87.035) (width 0.2) (layer "B.Cu") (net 9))
 (segment (start 192.305 66.715) (end 194.2067 66.715) (width 0.2) (layer "B.Cu") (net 9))
 (segment (start 193.2559 111.72) (end 192.305 111.72) (width 0.2) (layer "B.Cu") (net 9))
 (segment (start 194.2067 134.5167) (end 194.2067 132.04) (width 0.2) (layer "B.Cu") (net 9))
 (segment (start 197.585 87.035) (end 195.6833 87.035) (width 0.2) (layer "B.Cu") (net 9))
 (segment (start 198.5417 64.8133) (end 207.3783 55.9767) (width 0.2) (layer "B.Cu") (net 9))
 (segment (start 197.585 127.04) (end 195.6833 127.04) (width 0.2) (layer "B.Cu") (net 9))
 (segment (start 195.6833 127.04) (end 195.6833 130.5634) (width 0.2) (layer "B.Cu") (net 9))
 (segment (start 207.3783 55.9767) (end 207.3783 55.88) (width 0.2) (layer "B.Cu") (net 9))
 (segment (start 179.805 66.715) (end 192.305 66.715) (width 0.2) (layer "B.Cu") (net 9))
 (segment (start 193.2559 132.04) (end 192.305 132.04) (width 0.2) (layer "B.Cu") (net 9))
 (segment (start 192.205 87.075) (end 195.6433 87.075) (width 0.2) (layer "B.Cu") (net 9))
 (segment (start 193.2559 111.72) (end 194.2067 111.72) (width 0.2) (layer "B.Cu") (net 9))
 (segment (start 192.305 111.72) (end 179.805 111.72) (width 0.2) (layer "B.Cu") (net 9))
 (segment (start 193.2559 132.04) (end 194.2067 132.04) (width 0.2) (layer "B.Cu") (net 9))
 (segment (start 196.1084 64.8133) (end 198.5417 64.8133) (width 0.2) (layer "B.Cu") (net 9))
 (segment (start 197.685 111.76) (end 194.2467 111.76) (width 0.2) (layer "B.Cu") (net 9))
 (segment (start 208.28 55.88) (end 207.3783 55.88) (width 0.2) (layer "B.Cu") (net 9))
 (segment (start 203.835 144.145) (end 194.2067 134.5167) (width 0.2) (layer "B.Cu") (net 9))
 (segment (start 192.305 132.04) (end 179.805 132.04) (width 0.2) (layer "B.Cu") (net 9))
 (segment (start 197.585 127.04) (end 210.085 127.04) (width 0.2) (layer "B.Cu") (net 9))
 (segment (start 194.2467 111.76) (end 194.2067 111.72) (width 0.2) (layer "B.Cu") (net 9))
 (segment (start 179.705 87.075) (end 192.205 87.075) (width 0.2) (layer "B.Cu") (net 9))
 (segment (start 195.6833 130.5634) (end 194.2067 132.04) (width 0.2) (layer "B.Cu") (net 9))
 (segment (start 180.975 159.385) (end 176.7284 155.1384) (width 0.2) (layer "F.Cu") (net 22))
 (segment (start 176.7284 155.1384) (end 176.7284 78.1072) (width 0.2) (layer "F.Cu") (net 22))
 (via (at 176.7284 78.1072) (size 0.6) (drill 0.3) (layers "F.Cu" "B.Cu") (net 22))
 (segment (start 197.685 71.755) (end 195.7833 71.755) (width 0.2) (layer "B.Cu") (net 22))
 (segment (start 189.4311 78.1072) (end 195.7833 71.755) (width 0.2) (layer "B.Cu") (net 22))
 (segment (start 210.185 71.755) (end 197.685 71.755) (width 0.2) (layer "B.Cu") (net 22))
 (segment (start 176.7284 78.1072) (end 189.4311 78.1072) (width 0.2) (layer "B.Cu") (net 22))
 (segment (start 197.685 66.755) (end 199.5867 66.755) (width 0.2) (layer "F.Cu") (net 14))
 (segment (start 201.295 144.145) (end 201.295 68.4633) (width 0.2) (layer "F.Cu") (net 14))
 (segment (start 201.295 68.4633) (end 199.5867 66.755) (width 0.2) (layer "F.Cu") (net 14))
 (segment (start 210.185 66.755) (end 197.685 66.755) (width 0.2) (layer "B.Cu") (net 14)))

